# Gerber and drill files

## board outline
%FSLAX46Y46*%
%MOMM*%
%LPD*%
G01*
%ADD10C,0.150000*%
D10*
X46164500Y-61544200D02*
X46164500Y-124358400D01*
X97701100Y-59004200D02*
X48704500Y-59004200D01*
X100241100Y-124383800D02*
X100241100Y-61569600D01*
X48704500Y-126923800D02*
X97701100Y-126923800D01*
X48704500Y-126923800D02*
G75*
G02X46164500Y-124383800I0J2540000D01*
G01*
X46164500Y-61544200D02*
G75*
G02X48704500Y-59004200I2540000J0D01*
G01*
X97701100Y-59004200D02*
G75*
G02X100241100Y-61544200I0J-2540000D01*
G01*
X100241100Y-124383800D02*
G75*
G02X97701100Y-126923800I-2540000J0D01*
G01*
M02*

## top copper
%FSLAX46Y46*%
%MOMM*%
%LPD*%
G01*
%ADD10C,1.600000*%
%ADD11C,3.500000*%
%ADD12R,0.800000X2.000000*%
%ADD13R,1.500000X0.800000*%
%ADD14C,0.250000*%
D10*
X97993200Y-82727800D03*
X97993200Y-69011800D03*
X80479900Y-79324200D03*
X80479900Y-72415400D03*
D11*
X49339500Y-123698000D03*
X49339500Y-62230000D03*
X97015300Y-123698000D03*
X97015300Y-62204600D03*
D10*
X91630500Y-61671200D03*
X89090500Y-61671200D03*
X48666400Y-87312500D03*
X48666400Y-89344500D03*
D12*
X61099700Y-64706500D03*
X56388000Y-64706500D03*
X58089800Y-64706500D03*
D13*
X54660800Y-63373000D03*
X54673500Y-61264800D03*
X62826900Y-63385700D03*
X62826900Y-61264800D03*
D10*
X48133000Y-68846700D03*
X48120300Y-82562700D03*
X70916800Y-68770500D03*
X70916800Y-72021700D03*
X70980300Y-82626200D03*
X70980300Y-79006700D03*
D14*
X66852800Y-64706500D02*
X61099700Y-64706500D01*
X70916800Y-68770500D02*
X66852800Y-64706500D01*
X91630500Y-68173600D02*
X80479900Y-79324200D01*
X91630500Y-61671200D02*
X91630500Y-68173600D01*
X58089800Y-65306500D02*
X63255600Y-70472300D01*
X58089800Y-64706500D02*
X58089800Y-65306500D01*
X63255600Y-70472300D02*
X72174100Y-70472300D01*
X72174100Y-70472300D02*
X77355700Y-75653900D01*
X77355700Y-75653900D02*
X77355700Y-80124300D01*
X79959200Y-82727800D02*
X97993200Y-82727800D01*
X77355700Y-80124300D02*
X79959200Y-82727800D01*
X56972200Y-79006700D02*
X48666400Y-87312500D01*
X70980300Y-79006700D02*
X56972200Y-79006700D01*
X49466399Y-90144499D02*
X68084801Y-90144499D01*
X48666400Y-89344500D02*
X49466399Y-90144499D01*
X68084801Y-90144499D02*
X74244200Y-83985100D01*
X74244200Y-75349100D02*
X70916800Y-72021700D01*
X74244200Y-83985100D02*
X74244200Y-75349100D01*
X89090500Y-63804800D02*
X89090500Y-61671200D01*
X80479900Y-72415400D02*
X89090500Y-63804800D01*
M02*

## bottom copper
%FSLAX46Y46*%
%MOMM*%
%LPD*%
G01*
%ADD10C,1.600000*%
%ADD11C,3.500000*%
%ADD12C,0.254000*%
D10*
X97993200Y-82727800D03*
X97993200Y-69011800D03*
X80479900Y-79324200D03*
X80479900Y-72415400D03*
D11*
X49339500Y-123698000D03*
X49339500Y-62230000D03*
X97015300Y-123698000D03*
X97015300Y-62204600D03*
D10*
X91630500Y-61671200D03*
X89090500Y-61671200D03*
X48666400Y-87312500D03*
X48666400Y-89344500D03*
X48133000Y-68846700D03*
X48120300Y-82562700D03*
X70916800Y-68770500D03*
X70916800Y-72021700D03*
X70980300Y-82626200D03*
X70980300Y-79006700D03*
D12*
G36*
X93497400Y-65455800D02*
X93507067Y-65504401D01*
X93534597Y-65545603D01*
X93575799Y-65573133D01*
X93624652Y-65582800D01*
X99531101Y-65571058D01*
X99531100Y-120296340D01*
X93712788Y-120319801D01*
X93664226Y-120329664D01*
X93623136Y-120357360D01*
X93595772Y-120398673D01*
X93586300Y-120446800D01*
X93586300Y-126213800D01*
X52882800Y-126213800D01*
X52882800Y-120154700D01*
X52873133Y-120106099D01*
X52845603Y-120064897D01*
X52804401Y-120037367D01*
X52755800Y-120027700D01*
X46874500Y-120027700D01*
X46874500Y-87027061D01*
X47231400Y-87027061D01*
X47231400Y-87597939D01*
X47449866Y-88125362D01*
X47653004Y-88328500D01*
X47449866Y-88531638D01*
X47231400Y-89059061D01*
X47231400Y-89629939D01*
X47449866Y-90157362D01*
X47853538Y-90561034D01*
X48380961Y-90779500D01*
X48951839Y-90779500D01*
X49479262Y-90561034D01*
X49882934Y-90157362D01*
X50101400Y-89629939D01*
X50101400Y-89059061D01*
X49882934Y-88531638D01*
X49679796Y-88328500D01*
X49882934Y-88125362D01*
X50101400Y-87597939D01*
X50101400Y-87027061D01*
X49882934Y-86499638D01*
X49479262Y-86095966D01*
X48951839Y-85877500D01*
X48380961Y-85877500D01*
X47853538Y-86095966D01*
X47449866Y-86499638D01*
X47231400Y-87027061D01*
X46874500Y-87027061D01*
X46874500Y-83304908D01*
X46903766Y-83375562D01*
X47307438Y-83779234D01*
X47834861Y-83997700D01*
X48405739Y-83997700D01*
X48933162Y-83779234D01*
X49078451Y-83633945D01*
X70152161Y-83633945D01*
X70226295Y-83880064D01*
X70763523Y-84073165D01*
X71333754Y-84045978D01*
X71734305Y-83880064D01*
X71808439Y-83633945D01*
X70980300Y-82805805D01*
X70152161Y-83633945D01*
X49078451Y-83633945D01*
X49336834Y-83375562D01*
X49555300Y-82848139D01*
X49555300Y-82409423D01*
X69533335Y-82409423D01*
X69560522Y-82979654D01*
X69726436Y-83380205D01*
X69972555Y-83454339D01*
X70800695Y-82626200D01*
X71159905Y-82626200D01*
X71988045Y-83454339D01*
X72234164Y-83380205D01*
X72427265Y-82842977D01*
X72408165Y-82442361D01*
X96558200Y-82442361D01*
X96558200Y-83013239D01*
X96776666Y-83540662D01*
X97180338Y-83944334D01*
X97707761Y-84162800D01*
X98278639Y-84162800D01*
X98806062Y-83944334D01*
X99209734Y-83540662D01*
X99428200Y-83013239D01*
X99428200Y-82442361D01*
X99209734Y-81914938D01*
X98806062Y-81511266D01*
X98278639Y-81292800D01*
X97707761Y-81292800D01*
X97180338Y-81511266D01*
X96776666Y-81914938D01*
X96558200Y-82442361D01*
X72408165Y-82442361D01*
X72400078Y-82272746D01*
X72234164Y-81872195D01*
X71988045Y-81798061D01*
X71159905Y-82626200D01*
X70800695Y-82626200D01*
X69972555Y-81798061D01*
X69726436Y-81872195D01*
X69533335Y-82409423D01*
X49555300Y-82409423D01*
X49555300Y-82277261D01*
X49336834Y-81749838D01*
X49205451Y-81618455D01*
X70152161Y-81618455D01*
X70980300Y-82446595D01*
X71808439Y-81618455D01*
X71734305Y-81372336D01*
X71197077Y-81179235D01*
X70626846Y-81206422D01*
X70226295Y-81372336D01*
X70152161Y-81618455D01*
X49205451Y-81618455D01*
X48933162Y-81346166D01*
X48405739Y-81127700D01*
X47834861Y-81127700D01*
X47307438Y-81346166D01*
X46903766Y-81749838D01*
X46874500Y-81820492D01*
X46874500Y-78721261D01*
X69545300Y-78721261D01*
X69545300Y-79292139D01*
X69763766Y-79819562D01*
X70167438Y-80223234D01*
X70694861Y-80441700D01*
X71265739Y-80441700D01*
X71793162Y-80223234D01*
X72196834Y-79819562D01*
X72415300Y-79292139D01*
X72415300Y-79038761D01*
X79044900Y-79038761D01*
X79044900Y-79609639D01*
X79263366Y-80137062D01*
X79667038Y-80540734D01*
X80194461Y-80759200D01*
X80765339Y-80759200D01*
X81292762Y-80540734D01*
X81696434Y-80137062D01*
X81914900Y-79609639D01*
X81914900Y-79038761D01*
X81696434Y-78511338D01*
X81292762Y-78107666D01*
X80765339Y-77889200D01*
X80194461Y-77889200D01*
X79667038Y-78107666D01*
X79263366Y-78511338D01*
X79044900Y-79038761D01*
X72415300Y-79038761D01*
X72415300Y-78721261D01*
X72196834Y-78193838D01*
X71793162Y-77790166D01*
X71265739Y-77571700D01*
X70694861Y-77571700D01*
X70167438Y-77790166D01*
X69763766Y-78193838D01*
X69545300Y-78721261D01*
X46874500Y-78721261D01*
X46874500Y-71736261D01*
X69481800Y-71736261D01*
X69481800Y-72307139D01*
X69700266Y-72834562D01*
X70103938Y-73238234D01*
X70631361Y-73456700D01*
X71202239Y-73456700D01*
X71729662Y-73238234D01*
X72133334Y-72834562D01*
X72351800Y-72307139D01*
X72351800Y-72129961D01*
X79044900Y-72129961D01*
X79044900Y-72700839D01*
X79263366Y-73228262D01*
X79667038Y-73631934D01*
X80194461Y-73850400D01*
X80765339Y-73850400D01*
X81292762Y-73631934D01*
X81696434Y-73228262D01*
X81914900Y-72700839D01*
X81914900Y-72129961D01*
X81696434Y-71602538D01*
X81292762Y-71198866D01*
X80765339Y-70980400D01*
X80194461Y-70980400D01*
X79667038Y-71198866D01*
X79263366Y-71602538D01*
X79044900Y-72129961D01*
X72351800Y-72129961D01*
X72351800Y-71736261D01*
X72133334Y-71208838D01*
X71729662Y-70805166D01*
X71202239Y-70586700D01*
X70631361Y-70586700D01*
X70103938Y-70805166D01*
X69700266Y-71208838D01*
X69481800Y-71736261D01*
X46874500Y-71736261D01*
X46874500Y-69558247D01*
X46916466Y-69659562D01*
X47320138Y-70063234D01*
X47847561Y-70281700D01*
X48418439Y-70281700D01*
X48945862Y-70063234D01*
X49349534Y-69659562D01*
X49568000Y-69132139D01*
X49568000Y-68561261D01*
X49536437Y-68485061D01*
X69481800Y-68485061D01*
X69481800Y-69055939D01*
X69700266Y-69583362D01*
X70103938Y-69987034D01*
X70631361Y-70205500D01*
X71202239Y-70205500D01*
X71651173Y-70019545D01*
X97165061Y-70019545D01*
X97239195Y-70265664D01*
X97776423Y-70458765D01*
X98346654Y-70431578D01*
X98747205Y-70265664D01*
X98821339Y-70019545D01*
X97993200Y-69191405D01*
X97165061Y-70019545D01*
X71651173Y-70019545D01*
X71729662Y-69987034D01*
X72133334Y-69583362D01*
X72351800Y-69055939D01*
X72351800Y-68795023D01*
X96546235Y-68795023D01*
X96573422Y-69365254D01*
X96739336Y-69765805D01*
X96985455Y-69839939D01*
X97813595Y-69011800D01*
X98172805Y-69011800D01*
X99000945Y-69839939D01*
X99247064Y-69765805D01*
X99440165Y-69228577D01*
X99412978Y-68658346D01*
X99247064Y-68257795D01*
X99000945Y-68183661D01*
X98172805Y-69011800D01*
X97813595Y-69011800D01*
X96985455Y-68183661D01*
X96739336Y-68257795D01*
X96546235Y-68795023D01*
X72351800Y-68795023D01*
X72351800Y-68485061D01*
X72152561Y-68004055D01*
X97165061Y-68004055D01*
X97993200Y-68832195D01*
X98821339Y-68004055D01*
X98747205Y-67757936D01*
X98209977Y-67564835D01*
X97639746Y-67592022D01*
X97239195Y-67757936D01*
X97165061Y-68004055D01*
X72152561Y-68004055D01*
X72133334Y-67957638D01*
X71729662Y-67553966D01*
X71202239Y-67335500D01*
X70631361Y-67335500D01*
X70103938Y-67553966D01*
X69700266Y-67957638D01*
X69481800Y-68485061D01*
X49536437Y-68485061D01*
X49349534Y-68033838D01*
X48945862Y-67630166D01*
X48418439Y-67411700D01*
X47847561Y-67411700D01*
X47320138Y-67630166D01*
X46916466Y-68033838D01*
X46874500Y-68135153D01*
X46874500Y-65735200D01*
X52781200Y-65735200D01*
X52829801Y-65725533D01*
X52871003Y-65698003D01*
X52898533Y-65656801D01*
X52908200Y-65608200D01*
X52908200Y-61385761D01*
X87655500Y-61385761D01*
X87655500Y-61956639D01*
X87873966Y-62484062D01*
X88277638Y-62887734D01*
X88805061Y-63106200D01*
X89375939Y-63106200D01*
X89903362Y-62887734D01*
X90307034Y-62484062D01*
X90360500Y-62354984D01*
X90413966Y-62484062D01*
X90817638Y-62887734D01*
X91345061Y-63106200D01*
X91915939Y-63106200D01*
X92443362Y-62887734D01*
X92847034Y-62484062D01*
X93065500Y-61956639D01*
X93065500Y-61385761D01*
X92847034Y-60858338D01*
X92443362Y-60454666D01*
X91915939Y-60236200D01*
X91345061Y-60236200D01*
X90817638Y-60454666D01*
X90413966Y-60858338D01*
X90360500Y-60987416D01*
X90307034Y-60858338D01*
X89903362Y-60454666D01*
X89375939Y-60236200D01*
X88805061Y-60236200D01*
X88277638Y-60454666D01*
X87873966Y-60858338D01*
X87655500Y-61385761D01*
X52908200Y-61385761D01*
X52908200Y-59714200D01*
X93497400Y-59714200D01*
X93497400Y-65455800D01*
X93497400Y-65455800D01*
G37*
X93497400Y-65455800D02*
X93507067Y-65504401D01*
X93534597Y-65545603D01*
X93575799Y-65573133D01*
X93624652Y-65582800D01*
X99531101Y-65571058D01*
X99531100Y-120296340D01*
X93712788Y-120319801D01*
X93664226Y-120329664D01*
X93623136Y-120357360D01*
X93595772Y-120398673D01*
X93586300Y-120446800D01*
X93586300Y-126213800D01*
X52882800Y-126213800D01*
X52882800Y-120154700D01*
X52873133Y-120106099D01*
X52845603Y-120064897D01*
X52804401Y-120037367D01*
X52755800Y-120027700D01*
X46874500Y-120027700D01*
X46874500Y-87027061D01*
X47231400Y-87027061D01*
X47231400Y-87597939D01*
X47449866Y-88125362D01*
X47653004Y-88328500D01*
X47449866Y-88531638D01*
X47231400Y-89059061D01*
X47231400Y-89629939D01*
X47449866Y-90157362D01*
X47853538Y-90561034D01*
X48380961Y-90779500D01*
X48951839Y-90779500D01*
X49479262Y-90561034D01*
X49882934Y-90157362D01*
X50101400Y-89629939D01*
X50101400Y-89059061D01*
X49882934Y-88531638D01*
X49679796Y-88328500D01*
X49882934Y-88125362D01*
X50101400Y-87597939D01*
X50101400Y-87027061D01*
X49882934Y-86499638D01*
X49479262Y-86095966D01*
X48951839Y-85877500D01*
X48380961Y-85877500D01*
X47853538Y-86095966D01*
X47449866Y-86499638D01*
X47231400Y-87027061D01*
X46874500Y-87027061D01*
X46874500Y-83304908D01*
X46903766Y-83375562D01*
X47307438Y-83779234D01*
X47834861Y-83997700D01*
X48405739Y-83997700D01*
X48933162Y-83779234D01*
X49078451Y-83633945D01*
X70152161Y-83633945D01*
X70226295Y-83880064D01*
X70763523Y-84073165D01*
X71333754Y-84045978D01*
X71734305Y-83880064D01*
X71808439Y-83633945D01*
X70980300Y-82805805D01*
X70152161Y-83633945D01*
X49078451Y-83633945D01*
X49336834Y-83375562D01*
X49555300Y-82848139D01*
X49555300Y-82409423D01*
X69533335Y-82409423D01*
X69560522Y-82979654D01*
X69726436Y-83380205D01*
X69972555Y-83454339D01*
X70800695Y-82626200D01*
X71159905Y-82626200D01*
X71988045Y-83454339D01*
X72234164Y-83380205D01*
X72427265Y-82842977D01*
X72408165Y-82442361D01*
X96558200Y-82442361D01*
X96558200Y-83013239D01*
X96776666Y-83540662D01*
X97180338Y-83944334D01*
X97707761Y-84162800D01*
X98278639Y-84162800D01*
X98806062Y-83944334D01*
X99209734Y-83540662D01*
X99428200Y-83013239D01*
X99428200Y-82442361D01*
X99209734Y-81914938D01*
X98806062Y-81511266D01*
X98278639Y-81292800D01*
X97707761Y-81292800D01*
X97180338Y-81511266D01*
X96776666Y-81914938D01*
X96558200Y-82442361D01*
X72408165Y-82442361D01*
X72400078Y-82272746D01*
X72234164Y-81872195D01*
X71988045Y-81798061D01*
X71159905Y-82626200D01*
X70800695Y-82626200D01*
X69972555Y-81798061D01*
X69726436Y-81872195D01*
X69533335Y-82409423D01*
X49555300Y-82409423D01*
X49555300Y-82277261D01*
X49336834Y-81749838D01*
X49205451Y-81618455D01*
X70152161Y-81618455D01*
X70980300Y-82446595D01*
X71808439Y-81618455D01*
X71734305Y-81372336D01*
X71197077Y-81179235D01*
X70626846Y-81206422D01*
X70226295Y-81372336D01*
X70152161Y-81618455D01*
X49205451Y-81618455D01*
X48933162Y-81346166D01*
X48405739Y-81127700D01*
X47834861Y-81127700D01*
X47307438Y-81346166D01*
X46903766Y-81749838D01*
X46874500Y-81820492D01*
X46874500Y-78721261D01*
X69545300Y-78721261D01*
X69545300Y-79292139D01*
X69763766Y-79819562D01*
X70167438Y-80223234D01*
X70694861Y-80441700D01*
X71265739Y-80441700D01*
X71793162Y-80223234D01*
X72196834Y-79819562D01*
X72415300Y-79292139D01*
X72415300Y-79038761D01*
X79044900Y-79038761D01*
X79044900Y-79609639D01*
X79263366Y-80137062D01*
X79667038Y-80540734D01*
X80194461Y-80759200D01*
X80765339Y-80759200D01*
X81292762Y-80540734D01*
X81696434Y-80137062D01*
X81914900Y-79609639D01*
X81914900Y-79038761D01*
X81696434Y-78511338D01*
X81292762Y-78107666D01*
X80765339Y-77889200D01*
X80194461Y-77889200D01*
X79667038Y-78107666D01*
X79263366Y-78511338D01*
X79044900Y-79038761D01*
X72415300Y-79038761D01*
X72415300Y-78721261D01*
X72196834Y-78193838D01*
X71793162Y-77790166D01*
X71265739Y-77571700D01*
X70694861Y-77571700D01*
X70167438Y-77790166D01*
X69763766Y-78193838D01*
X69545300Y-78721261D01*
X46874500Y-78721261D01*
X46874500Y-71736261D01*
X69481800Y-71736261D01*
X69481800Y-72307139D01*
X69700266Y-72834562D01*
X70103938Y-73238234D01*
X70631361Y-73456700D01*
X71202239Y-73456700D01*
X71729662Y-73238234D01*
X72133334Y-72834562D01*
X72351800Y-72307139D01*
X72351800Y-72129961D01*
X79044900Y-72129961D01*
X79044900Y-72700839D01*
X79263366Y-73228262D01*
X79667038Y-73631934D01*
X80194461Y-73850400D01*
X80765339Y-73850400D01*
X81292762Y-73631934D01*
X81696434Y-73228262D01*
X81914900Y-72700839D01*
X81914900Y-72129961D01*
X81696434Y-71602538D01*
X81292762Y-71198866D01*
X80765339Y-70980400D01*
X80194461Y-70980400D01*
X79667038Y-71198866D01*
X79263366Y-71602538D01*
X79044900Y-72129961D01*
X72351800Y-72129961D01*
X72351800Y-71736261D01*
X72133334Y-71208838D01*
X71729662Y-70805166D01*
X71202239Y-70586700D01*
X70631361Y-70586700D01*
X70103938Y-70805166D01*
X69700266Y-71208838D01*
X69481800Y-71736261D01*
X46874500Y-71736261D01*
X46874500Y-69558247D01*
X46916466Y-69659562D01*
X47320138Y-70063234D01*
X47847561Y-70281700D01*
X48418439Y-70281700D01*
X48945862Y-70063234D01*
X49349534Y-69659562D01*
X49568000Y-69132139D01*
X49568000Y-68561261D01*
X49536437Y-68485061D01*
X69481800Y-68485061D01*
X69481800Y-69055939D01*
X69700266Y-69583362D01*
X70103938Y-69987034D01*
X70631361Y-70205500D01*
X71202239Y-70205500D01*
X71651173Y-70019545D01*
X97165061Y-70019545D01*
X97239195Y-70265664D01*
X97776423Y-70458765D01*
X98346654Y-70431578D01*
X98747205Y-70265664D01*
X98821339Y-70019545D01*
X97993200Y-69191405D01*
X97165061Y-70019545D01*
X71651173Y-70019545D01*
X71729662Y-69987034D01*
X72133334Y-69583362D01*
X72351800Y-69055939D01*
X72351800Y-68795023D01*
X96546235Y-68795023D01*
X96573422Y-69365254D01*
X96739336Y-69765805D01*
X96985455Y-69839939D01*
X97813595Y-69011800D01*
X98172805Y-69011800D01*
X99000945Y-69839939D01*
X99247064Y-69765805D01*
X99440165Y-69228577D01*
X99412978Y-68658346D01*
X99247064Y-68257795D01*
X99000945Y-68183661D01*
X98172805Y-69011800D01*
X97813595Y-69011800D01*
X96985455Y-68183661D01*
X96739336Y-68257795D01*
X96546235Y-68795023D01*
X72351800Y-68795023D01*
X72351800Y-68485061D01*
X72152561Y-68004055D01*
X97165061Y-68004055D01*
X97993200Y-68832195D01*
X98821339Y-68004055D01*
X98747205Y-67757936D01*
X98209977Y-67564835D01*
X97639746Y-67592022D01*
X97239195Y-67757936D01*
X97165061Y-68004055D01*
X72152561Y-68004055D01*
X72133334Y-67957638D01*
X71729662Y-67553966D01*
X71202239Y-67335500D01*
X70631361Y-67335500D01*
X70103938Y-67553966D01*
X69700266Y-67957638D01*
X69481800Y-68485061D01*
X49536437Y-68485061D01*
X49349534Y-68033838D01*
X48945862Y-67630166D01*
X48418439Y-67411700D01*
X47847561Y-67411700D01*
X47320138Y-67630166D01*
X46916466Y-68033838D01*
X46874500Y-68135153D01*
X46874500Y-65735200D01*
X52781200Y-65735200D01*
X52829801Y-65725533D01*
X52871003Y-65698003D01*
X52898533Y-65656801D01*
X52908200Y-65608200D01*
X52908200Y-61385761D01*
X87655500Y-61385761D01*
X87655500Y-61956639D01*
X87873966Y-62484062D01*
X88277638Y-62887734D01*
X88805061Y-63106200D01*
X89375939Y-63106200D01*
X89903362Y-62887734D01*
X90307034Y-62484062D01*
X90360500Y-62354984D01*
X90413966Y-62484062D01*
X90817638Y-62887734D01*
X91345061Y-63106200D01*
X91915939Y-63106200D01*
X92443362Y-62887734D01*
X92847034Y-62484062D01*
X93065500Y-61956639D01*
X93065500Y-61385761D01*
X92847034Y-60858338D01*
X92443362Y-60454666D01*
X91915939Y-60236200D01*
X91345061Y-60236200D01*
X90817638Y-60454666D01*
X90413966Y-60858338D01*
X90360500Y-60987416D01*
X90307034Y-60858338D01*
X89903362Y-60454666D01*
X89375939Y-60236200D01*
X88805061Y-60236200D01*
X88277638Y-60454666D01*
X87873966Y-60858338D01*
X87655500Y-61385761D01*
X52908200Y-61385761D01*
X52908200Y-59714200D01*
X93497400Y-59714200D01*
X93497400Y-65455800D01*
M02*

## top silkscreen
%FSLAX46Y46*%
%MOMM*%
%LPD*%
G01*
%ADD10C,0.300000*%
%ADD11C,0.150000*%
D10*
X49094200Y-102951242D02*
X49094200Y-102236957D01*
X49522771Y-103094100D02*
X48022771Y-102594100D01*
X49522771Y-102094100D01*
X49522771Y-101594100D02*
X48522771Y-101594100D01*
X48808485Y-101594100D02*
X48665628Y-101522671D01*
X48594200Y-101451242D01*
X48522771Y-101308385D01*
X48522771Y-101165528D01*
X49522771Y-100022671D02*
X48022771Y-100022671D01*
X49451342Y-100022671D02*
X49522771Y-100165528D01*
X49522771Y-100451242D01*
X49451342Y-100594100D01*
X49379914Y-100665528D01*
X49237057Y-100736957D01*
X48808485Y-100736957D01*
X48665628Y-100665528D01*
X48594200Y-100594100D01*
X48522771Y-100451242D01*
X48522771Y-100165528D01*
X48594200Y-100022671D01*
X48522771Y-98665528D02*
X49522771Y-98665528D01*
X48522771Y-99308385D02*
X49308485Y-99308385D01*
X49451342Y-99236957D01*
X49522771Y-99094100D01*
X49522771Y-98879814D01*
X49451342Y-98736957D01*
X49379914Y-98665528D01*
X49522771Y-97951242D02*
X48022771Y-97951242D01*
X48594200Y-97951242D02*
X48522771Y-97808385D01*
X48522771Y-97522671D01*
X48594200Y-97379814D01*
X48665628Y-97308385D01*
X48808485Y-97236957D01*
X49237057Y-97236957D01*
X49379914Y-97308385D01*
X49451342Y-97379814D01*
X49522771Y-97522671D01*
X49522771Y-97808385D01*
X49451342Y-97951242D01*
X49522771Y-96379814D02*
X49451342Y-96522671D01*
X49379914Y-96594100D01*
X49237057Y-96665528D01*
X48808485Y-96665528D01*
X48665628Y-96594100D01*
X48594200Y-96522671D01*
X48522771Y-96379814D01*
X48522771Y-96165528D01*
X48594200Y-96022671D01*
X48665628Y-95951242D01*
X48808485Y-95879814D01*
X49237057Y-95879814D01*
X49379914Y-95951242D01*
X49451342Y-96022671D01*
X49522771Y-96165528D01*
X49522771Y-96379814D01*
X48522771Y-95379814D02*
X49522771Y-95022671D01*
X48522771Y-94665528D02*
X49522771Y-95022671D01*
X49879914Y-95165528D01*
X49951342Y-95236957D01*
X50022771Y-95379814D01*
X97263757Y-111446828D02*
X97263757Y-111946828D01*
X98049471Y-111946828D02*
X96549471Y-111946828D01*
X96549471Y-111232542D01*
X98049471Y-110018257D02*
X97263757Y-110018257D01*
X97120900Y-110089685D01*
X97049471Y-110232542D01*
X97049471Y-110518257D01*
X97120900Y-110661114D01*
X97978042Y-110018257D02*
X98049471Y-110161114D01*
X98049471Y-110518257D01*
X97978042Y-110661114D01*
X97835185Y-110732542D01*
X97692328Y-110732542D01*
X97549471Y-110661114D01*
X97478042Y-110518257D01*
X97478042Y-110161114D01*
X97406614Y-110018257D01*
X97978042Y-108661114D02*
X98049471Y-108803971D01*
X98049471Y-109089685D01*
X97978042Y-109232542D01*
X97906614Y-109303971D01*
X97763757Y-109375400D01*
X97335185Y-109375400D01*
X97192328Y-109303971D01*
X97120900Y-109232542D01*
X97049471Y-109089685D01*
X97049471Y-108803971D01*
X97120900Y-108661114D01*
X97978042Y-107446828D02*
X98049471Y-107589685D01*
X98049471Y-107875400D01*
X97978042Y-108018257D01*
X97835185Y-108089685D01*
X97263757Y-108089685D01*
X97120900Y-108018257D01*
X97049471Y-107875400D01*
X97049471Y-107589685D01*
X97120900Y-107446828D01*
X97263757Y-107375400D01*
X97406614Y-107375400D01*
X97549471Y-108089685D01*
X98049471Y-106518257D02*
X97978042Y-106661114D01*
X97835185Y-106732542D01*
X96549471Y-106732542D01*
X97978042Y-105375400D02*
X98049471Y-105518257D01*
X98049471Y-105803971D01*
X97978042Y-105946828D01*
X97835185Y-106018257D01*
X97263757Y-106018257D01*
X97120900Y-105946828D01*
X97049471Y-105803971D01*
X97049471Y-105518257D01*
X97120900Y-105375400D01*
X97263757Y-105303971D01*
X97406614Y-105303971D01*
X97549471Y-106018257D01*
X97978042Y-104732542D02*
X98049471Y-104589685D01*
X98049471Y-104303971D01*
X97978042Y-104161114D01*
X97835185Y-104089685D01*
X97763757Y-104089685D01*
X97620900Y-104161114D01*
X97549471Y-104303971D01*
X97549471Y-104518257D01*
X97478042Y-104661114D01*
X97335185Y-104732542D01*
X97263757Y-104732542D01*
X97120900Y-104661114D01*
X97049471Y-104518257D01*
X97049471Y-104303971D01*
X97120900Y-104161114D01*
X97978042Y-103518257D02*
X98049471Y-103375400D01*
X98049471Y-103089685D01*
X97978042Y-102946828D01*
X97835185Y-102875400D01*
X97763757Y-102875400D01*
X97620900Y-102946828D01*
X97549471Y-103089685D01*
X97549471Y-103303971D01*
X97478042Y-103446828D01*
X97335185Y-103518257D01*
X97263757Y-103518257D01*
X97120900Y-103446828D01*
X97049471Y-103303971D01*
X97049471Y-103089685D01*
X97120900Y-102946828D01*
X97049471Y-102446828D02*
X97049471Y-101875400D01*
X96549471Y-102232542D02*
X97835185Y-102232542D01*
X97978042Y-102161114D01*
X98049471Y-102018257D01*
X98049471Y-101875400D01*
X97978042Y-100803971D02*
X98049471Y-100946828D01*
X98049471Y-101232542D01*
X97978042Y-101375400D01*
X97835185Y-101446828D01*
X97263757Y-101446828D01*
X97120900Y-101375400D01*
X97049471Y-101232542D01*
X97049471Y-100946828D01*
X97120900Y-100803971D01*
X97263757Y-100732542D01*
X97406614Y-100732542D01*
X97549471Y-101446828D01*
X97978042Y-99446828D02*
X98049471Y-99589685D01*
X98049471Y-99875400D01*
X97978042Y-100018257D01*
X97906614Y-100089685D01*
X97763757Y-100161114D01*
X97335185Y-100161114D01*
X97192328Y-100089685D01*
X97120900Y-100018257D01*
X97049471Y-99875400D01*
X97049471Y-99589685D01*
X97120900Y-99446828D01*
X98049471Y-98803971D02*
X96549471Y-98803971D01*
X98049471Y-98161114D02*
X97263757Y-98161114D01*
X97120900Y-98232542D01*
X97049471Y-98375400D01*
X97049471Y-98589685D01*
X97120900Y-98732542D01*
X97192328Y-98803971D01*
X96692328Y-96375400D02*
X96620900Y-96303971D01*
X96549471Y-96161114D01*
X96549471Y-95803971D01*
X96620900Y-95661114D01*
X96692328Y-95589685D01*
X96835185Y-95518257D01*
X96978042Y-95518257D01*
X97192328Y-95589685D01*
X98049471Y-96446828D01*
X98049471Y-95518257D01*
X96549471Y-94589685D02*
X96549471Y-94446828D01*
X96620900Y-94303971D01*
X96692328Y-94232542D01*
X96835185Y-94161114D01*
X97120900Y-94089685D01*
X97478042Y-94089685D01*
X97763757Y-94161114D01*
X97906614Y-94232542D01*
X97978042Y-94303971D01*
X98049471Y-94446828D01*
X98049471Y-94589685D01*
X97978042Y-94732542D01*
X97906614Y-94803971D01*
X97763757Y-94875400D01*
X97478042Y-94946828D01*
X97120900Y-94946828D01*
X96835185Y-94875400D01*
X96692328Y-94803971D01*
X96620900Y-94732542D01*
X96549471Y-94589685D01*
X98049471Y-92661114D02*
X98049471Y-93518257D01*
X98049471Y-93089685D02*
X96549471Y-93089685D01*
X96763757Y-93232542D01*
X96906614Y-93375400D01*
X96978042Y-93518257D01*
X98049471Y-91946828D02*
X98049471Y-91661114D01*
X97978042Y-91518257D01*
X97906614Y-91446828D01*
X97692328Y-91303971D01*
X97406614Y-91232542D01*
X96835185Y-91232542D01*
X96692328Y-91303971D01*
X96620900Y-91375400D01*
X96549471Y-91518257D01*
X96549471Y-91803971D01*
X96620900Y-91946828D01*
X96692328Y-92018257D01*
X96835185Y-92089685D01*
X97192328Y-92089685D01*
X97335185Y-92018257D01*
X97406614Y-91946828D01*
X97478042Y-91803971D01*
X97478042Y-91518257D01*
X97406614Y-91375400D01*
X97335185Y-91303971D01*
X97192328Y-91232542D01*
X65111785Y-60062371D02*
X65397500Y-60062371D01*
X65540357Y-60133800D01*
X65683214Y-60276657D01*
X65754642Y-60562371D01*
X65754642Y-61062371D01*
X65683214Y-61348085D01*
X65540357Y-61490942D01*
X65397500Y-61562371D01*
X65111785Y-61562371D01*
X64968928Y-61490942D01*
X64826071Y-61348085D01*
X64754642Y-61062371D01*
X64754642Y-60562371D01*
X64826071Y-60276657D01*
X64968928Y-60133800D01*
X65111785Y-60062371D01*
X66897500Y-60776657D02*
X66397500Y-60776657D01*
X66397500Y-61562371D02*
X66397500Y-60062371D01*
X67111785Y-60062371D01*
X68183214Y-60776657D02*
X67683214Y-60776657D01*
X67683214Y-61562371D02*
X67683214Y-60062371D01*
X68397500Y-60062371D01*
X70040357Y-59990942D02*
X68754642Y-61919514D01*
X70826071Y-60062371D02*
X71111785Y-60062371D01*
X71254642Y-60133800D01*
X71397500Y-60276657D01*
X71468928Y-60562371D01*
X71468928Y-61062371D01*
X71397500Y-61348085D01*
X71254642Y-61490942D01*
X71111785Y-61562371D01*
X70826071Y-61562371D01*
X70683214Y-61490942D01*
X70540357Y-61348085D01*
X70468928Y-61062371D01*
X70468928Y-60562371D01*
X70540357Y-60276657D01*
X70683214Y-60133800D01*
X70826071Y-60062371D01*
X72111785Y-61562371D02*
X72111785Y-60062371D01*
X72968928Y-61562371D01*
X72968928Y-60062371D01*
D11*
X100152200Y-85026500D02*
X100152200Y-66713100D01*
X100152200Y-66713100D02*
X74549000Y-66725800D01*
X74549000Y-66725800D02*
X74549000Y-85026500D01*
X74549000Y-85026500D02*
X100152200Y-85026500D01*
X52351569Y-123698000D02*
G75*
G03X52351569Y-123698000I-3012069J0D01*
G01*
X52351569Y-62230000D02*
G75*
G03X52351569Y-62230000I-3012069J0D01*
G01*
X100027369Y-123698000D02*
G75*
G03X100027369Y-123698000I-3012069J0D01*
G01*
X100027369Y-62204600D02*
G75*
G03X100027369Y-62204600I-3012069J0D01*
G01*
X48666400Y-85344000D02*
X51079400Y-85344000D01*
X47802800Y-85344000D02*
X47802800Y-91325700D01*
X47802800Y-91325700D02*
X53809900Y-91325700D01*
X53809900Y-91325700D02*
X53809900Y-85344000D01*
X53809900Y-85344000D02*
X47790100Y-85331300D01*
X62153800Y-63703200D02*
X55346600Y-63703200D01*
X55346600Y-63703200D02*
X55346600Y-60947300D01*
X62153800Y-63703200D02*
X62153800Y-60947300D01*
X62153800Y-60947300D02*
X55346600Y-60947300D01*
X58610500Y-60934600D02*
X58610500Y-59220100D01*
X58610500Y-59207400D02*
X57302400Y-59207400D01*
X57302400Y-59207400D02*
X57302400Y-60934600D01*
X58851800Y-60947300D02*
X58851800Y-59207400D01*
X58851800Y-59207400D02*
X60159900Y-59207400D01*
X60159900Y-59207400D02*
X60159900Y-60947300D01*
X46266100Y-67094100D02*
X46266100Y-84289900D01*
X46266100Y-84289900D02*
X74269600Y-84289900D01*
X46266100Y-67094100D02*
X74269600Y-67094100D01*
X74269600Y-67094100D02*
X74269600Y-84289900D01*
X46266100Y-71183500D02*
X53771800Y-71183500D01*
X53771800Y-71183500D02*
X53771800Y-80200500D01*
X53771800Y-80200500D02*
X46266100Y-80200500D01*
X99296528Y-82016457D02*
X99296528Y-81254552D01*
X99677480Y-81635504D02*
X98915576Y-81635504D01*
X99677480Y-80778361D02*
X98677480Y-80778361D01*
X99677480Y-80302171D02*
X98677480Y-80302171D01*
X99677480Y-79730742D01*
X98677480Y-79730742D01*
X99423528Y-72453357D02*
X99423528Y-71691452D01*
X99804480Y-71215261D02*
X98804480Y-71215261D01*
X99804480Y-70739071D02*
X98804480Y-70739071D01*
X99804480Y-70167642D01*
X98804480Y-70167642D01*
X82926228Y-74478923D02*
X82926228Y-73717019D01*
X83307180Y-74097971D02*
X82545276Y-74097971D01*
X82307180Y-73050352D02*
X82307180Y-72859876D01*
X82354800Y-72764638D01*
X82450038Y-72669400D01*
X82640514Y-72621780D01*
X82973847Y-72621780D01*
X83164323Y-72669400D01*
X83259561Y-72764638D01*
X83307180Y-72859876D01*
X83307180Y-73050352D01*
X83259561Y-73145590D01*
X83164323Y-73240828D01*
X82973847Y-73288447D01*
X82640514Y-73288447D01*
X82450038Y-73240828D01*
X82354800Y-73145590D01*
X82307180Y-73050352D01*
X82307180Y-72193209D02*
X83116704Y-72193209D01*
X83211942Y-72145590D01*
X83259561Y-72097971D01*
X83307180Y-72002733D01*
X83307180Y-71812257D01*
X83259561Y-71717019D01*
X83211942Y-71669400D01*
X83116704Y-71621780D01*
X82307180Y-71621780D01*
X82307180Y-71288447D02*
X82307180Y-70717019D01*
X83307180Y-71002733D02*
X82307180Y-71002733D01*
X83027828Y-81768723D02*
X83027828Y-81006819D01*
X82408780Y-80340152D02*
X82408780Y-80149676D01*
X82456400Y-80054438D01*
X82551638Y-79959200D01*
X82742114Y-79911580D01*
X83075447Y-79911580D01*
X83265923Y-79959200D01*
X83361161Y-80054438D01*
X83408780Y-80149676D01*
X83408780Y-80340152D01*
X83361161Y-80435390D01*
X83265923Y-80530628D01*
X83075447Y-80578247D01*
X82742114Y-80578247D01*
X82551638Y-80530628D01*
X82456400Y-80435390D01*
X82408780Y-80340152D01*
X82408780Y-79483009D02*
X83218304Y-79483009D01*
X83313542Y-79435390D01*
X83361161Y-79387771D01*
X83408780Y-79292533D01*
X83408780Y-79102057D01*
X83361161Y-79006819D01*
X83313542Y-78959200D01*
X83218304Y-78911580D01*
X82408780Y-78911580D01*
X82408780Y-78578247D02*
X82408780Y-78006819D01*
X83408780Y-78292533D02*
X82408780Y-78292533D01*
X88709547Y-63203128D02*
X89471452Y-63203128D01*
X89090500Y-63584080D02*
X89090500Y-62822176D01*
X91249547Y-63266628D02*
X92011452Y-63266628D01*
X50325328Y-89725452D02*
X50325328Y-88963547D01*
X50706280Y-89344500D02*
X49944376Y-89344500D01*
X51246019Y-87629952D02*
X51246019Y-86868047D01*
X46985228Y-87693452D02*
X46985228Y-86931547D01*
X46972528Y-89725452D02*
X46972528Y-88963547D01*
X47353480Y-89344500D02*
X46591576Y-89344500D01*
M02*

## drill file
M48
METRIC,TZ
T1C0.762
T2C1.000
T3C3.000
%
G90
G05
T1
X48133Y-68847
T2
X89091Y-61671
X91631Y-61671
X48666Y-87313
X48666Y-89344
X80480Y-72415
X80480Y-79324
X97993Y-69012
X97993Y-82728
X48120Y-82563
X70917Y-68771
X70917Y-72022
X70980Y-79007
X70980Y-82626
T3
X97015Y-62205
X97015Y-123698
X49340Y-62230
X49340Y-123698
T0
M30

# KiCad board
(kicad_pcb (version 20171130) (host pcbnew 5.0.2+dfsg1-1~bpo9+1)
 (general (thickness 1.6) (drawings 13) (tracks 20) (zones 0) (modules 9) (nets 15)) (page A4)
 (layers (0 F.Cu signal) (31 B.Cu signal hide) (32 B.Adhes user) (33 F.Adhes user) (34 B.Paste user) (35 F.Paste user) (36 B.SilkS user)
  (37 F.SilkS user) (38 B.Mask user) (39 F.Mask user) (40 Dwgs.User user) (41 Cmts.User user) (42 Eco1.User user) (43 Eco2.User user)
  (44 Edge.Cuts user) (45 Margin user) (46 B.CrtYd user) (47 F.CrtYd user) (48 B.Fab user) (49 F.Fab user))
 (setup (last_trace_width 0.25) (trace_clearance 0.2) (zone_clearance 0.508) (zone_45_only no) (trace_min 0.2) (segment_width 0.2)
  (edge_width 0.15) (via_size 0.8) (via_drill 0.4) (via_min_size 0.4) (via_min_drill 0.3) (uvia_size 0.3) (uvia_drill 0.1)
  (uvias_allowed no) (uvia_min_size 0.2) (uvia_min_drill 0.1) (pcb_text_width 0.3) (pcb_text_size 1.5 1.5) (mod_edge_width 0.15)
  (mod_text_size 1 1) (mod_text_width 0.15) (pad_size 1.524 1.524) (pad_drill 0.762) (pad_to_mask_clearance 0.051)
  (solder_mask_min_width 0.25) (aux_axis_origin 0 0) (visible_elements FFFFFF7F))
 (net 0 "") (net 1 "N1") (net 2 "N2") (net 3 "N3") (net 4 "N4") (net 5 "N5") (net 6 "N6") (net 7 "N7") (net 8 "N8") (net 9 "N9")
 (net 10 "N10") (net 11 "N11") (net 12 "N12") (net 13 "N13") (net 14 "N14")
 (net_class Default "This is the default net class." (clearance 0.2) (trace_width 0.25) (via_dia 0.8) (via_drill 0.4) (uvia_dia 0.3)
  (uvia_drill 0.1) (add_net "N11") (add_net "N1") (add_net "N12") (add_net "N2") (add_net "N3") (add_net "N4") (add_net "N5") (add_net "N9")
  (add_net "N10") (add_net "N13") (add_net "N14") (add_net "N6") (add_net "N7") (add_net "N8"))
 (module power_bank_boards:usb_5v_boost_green (layer F.Cu) (at 97.9932 75.8698 90)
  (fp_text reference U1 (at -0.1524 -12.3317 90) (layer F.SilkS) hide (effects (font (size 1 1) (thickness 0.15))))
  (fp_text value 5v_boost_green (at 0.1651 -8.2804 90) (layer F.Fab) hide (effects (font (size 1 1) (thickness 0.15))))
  (fp_line (start -9.1567 2.159) (end 9.1567 2.159) (layer F.SilkS) (width 0.15))
  (fp_line (start 9.1567 2.159) (end 9.144 -23.4442) (layer F.SilkS) (width 0.15))
  (fp_line (start 9.144 -23.4442) (end -9.1567 -23.4442) (layer F.SilkS) (width 0.15))
  (fp_line (start -9.1567 -23.4442) (end -9.1567 2.159) (layer F.SilkS) (width 0.15))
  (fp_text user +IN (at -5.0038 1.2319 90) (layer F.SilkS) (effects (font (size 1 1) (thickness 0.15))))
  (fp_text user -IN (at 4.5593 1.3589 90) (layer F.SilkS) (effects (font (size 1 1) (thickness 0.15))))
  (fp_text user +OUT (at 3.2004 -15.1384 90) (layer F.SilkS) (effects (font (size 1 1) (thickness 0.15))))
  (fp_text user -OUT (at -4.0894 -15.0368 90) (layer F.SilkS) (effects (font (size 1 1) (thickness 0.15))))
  (pad 1 thru_hole circle (at -6.858 0 90) (size 1.6 1.6) (drill 1) (layers *.Cu *.Mask) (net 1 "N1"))
  (pad 2 thru_hole circle (at 6.858 0 90) (size 1.6 1.6) (drill 1) (layers *.Cu *.Mask) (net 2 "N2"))
  (pad 3 thru_hole circle (at -3.4544 -17.5133 90) (size 1.6 1.6) (drill 1) (layers *.Cu *.Mask) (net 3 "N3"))
  (pad 4 thru_hole circle (at 3.4544 -17.5133 90) (size 1.6 1.6) (drill 1) (layers *.Cu *.Mask) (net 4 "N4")))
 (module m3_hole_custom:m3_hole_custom (layer F.Cu) (at 49.3395 123.698)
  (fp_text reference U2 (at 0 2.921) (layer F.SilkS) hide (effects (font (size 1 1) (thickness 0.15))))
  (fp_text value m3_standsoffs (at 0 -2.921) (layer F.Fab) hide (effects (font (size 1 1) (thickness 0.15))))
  (fp_circle (center 0 0) (end 2.8575 0.9525) (layer F.SilkS) (width 0.15))
  (pad 1 thru_hole circle (at 0 0) (size 3.5 3.5) (drill 3) (layers *.Cu *.Mask) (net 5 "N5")))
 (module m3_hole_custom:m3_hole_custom (layer F.Cu) (at 49.3395 62.23)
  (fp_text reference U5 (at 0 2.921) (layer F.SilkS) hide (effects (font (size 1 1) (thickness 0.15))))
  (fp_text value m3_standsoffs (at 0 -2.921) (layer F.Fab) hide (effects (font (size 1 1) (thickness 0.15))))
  (fp_circle (center 0 0) (end 2.8575 0.9525) (layer F.SilkS) (width 0.15))
  (pad 1 thru_hole circle (at 0 0) (size 3.5 3.5) (drill 3) (layers *.Cu *.Mask) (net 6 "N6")))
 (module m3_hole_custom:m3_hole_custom (layer F.Cu) (at 97.0153 123.698)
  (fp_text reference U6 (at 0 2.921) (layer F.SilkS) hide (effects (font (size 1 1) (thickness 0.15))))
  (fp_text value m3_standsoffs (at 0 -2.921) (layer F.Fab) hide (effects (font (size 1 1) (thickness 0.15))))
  (fp_circle (center 0 0) (end 2.8575 0.9525) (layer F.SilkS) (width 0.15))
  (pad 1 thru_hole circle (at 0 0) (size 3.5 3.5) (drill 3) (layers *.Cu *.Mask) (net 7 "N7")))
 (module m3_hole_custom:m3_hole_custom (layer F.Cu) (at 97.0153 62.2046)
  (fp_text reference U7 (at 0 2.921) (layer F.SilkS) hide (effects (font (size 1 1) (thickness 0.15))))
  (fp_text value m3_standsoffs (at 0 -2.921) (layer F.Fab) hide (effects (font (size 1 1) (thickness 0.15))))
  (fp_circle (center 0 0) (end 2.8575 0.9525) (layer F.SilkS) (width 0.15))
  (pad 1 thru_hole circle (at 0 0) (size 3.5 3.5) (drill 3) (layers *.Cu *.Mask) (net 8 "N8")))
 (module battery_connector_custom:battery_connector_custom (layer F.Cu) (at 90.3605 61.6712 180)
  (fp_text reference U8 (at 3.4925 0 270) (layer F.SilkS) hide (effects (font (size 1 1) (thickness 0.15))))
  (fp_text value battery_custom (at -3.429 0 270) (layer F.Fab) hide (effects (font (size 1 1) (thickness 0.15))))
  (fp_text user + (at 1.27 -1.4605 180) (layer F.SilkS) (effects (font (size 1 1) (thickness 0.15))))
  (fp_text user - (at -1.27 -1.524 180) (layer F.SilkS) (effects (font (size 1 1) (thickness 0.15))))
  (pad 1 thru_hole circle (at -1.27 0 180) (size 1.6 1.6) (drill 1) (layers *.Cu *.Mask) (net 3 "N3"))
  (pad 2 thru_hole circle (at 1.27 0 180) (size 1.6 1.6) (drill 1) (layers *.Cu *.Mask) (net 4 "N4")))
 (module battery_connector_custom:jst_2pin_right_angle (layer F.Cu) (at 48.6664 88.3285 270)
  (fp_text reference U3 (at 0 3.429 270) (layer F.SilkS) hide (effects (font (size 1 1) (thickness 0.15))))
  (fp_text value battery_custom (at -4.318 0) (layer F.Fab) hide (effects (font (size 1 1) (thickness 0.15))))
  (fp_line (start -2.9845 0) (end -2.9845 -2.413) (layer F.SilkS) (width 0.15))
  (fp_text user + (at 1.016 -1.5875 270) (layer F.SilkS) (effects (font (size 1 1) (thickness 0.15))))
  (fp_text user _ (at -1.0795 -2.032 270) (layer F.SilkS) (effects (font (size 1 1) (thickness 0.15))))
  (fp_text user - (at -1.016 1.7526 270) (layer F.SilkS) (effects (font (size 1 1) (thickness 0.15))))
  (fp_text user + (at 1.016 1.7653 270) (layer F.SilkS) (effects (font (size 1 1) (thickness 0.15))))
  (fp_line (start -2.9845 0.8636) (end 2.9972 0.8636) (layer F.SilkS) (width 0.15))
  (fp_line (start 2.9972 0.8636) (end 2.9972 -5.1435) (layer F.SilkS) (width 0.15))
  (fp_line (start 2.9972 -5.1435) (end -2.9845 -5.1435) (layer F.SilkS) (width 0.15))
  (fp_line (start -2.9845 -5.1435) (end -2.9972 0.8763) (layer F.SilkS) (width 0.15))
  (pad 1 thru_hole circle (at -1.016 0 270) (size 1.6 1.6) (drill 1) (layers *.Cu *.Mask) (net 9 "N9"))
  (pad 2 thru_hole circle (at 1.016 0 270) (size 1.6 1.6) (drill 1) (layers *.Cu *.Mask) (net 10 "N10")))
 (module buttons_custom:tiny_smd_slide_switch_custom (layer F.Cu) (at 61.0997 63.7032 180)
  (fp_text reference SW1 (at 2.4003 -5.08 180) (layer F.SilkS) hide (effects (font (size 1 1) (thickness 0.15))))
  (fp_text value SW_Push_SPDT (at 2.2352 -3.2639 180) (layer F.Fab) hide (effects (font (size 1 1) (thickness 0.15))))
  (fp_line (start -1.0541 0) (end 5.7531 0) (layer F.SilkS) (width 0.15))
  (fp_line (start 5.7531 0) (end 5.7531 2.7559) (layer F.SilkS) (width 0.15))
  (fp_line (start -1.0541 0) (end -1.0541 2.7559) (layer F.SilkS) (width 0.15))
  (fp_line (start -1.0541 2.7559) (end 5.7531 2.7559) (layer F.SilkS) (width 0.15))
  (fp_line (start 2.4892 2.7686) (end 2.4892 4.4831) (layer F.SilkS) (width 0.15))
  (fp_line (start 2.4892 4.4958) (end 3.7973 4.4958) (layer F.SilkS) (width 0.15))
  (fp_line (start 3.7973 4.4958) (end 3.7973 2.7686) (layer F.SilkS) (width 0.15))
  (fp_line (start 2.2479 2.7559) (end 2.2479 4.4958) (layer F.SilkS) (width 0.15))
  (fp_line (start 2.2479 4.4958) (end 0.9398 4.4958) (layer F.SilkS) (width 0.15))
  (fp_line (start 0.9398 4.4958) (end 0.9398 2.7559) (layer F.SilkS) (width 0.15))
  (pad 1 smd rect (at 0 -1.0033 180) (size 0.8 2) (layers F.Cu F.Paste F.Mask) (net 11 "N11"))
  (pad 3 smd rect (at 4.7117 -1.0033 180) (size 0.8 2) (layers F.Cu F.Paste F.Mask) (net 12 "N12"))
  (pad 2 smd rect (at 3.0099 -1.0033 180) (size 0.8 2) (layers F.Cu F.Paste F.Mask) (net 1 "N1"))
  (pad 4 smd rect (at 6.4389 0.3302 270) (size 0.8 1.5) (layers F.Cu F.Paste F.Mask))
  (pad 4 smd rect (at 6.4262 2.4384 270) (size 0.8 1.5) (layers F.Cu F.Paste F.Mask))
  (pad 4 smd rect (at -1.7272 0.3175 270) (size 0.8 1.5) (layers F.Cu F.Paste F.Mask))
  (pad 4 smd rect (at -1.7272 2.4384 270) (size 0.8 1.5) (layers F.Cu F.Paste F.Mask)))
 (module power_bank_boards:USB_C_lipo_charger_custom (layer F.Cu) (at 48.133 75.692 270)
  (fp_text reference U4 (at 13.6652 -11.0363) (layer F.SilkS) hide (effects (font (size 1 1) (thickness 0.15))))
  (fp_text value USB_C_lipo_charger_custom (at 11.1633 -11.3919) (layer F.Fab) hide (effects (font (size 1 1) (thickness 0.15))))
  (fp_line (start -8.5979 1.8669) (end 8.5979 1.8669) (layer F.SilkS) (width 0.15))
  (fp_line (start 8.5979 1.8669) (end 8.5979 -26.1366) (layer F.SilkS) (width 0.15))
  (fp_line (start -8.5979 1.8669) (end -8.5979 -26.1366) (layer F.SilkS) (width 0.15))
  (fp_line (start -8.5979 -26.1366) (end 8.5979 -26.1366) (layer F.SilkS) (width 0.15))
  (fp_line (start -4.5085 1.8669) (end -4.5085 -5.6388) (layer F.SilkS) (width 0.15))
  (fp_line (start -4.5085 -5.6388) (end 4.5085 -5.6388) (layer F.SilkS) (width 0.15))
  (fp_line (start 4.5085 -5.6388) (end 4.5085 1.8669) (layer F.SilkS) (width 0.15))
  (pad 1 thru_hole circle (at -6.8453 0 270) (size 1.6 1.6) (drill 0.7621) (layers *.Cu *.Mask) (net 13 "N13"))
  (pad 2 thru_hole circle (at 6.8707 0.0127 270) (size 1.6 1.6) (drill 1) (layers *.Cu *.Mask) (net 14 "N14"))
  (pad 3 thru_hole circle (at -6.9215 -22.7838 270) (size 1.6 1.6) (drill 1) (layers *.Cu *.Mask) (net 11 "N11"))
  (pad 4 thru_hole circle (at -3.6703 -22.7838 270) (size 1.6 1.6) (drill 1) (layers *.Cu *.Mask) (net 10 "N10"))
  (pad 6 thru_hole circle (at 6.9342 -22.8473 270) (size 1.6 1.6) (drill 1) (layers *.Cu *.Mask) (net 2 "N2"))
  (pad 5 thru_hole circle (at 3.3147 -22.8473 270) (size 1.6 1.6) (drill 1) (layers *.Cu *.Mask) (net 9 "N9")))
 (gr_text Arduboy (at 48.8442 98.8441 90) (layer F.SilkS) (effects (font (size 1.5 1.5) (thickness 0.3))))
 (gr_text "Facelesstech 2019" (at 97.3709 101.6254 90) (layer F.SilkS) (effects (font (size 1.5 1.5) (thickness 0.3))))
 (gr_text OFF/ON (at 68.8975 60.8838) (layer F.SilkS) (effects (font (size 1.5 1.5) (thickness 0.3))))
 (gr_line (start 46.1645 61.5442) (end 46.1645 124.3584) (layer Edge.Cuts) (width 0.15))
 (gr_line (start 97.7011 59.0042) (end 48.7045 59.0042) (layer Edge.Cuts) (width 0.15))
 (gr_line (start 100.2411 124.3838) (end 100.2411 61.5696) (layer Edge.Cuts) (width 0.15))
 (gr_line (start 48.7045 126.9238) (end 97.7011 126.9238) (layer Edge.Cuts) (width 0.15))
 (gr_arc (start 48.7045 124.3838) (end 46.1645 124.3838) (angle -90) (layer Edge.Cuts) (width 0.15))
 (gr_arc (start 48.7045 61.5442) (end 48.7045 59.0042) (angle -90) (layer Edge.Cuts) (width 0.15))
 (gr_arc (start 97.7011 61.5442) (end 100.2411 61.5442) (angle -90) (layer Edge.Cuts) (width 0.15))
 (gr_arc (start 97.7011 124.3838) (end 97.7011 126.9238) (angle -90) (layer Edge.Cuts) (width 0.15))
 (segment (start 66.8528 64.7065) (end 61.0997 64.7065) (width 0.25) (layer F.Cu) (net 11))
 (segment (start 70.9168 68.7705) (end 66.8528 64.7065) (width 0.25) (layer F.Cu) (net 11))
 (segment (start 91.6305 68.1736) (end 80.4799 79.3242) (width 0.25) (layer F.Cu) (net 3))
 (segment (start 91.6305 61.6712) (end 91.6305 68.1736) (width 0.25) (layer F.Cu) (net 3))
 (segment (start 58.0898 65.3065) (end 63.2556 70.4723) (width 0.25) (layer F.Cu) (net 1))
 (segment (start 58.0898 64.7065) (end 58.0898 65.3065) (width 0.25) (layer F.Cu) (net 1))
 (segment (start 63.2556 70.4723) (end 72.1741 70.4723) (width 0.25) (layer F.Cu) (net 1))
 (segment (start 72.1741 70.4723) (end 77.3557 75.6539) (width 0.25) (layer F.Cu) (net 1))
 (segment (start 77.3557 75.6539) (end 77.3557 80.1243) (width 0.25) (layer F.Cu) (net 1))
 (segment (start 79.9592 82.7278) (end 97.9932 82.7278) (width 0.25) (layer F.Cu) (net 1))
 (segment (start 77.3557 80.1243) (end 79.9592 82.7278) (width 0.25) (layer F.Cu) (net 1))
 (segment (start 56.9722 79.0067) (end 48.6664 87.3125) (width 0.25) (layer F.Cu) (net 9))
 (segment (start 70.9803 79.0067) (end 56.9722 79.0067) (width 0.25) (layer F.Cu) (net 9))
 (segment (start 49.466399 90.144499) (end 68.084801 90.144499) (width 0.25) (layer F.Cu) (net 10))
 (segment (start 48.6664 89.3445) (end 49.466399 90.144499) (width 0.25) (layer F.Cu) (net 10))
 (segment (start 68.084801 90.144499) (end 74.2442 83.9851) (width 0.25) (layer F.Cu) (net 10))
 (segment (start 74.2442 75.3491) (end 70.9168 72.0217) (width 0.25) (layer F.Cu) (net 10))
 (segment (start 74.2442 83.9851) (end 74.2442 75.3491) (width 0.25) (layer F.Cu) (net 10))
 (segment (start 89.0905 63.8048) (end 89.0905 61.6712) (width 0.25) (layer F.Cu) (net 4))
 (segment (start 80.4799 72.4154) (end 89.0905 63.8048) (width 0.25) (layer F.Cu) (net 4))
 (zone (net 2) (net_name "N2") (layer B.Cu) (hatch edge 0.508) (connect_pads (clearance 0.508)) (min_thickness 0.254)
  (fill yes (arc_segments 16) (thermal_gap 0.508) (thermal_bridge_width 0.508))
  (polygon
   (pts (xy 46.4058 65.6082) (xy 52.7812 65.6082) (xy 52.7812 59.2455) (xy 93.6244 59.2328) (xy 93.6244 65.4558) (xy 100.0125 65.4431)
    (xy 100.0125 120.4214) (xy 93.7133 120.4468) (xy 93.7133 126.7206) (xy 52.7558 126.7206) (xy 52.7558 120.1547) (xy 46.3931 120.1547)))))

